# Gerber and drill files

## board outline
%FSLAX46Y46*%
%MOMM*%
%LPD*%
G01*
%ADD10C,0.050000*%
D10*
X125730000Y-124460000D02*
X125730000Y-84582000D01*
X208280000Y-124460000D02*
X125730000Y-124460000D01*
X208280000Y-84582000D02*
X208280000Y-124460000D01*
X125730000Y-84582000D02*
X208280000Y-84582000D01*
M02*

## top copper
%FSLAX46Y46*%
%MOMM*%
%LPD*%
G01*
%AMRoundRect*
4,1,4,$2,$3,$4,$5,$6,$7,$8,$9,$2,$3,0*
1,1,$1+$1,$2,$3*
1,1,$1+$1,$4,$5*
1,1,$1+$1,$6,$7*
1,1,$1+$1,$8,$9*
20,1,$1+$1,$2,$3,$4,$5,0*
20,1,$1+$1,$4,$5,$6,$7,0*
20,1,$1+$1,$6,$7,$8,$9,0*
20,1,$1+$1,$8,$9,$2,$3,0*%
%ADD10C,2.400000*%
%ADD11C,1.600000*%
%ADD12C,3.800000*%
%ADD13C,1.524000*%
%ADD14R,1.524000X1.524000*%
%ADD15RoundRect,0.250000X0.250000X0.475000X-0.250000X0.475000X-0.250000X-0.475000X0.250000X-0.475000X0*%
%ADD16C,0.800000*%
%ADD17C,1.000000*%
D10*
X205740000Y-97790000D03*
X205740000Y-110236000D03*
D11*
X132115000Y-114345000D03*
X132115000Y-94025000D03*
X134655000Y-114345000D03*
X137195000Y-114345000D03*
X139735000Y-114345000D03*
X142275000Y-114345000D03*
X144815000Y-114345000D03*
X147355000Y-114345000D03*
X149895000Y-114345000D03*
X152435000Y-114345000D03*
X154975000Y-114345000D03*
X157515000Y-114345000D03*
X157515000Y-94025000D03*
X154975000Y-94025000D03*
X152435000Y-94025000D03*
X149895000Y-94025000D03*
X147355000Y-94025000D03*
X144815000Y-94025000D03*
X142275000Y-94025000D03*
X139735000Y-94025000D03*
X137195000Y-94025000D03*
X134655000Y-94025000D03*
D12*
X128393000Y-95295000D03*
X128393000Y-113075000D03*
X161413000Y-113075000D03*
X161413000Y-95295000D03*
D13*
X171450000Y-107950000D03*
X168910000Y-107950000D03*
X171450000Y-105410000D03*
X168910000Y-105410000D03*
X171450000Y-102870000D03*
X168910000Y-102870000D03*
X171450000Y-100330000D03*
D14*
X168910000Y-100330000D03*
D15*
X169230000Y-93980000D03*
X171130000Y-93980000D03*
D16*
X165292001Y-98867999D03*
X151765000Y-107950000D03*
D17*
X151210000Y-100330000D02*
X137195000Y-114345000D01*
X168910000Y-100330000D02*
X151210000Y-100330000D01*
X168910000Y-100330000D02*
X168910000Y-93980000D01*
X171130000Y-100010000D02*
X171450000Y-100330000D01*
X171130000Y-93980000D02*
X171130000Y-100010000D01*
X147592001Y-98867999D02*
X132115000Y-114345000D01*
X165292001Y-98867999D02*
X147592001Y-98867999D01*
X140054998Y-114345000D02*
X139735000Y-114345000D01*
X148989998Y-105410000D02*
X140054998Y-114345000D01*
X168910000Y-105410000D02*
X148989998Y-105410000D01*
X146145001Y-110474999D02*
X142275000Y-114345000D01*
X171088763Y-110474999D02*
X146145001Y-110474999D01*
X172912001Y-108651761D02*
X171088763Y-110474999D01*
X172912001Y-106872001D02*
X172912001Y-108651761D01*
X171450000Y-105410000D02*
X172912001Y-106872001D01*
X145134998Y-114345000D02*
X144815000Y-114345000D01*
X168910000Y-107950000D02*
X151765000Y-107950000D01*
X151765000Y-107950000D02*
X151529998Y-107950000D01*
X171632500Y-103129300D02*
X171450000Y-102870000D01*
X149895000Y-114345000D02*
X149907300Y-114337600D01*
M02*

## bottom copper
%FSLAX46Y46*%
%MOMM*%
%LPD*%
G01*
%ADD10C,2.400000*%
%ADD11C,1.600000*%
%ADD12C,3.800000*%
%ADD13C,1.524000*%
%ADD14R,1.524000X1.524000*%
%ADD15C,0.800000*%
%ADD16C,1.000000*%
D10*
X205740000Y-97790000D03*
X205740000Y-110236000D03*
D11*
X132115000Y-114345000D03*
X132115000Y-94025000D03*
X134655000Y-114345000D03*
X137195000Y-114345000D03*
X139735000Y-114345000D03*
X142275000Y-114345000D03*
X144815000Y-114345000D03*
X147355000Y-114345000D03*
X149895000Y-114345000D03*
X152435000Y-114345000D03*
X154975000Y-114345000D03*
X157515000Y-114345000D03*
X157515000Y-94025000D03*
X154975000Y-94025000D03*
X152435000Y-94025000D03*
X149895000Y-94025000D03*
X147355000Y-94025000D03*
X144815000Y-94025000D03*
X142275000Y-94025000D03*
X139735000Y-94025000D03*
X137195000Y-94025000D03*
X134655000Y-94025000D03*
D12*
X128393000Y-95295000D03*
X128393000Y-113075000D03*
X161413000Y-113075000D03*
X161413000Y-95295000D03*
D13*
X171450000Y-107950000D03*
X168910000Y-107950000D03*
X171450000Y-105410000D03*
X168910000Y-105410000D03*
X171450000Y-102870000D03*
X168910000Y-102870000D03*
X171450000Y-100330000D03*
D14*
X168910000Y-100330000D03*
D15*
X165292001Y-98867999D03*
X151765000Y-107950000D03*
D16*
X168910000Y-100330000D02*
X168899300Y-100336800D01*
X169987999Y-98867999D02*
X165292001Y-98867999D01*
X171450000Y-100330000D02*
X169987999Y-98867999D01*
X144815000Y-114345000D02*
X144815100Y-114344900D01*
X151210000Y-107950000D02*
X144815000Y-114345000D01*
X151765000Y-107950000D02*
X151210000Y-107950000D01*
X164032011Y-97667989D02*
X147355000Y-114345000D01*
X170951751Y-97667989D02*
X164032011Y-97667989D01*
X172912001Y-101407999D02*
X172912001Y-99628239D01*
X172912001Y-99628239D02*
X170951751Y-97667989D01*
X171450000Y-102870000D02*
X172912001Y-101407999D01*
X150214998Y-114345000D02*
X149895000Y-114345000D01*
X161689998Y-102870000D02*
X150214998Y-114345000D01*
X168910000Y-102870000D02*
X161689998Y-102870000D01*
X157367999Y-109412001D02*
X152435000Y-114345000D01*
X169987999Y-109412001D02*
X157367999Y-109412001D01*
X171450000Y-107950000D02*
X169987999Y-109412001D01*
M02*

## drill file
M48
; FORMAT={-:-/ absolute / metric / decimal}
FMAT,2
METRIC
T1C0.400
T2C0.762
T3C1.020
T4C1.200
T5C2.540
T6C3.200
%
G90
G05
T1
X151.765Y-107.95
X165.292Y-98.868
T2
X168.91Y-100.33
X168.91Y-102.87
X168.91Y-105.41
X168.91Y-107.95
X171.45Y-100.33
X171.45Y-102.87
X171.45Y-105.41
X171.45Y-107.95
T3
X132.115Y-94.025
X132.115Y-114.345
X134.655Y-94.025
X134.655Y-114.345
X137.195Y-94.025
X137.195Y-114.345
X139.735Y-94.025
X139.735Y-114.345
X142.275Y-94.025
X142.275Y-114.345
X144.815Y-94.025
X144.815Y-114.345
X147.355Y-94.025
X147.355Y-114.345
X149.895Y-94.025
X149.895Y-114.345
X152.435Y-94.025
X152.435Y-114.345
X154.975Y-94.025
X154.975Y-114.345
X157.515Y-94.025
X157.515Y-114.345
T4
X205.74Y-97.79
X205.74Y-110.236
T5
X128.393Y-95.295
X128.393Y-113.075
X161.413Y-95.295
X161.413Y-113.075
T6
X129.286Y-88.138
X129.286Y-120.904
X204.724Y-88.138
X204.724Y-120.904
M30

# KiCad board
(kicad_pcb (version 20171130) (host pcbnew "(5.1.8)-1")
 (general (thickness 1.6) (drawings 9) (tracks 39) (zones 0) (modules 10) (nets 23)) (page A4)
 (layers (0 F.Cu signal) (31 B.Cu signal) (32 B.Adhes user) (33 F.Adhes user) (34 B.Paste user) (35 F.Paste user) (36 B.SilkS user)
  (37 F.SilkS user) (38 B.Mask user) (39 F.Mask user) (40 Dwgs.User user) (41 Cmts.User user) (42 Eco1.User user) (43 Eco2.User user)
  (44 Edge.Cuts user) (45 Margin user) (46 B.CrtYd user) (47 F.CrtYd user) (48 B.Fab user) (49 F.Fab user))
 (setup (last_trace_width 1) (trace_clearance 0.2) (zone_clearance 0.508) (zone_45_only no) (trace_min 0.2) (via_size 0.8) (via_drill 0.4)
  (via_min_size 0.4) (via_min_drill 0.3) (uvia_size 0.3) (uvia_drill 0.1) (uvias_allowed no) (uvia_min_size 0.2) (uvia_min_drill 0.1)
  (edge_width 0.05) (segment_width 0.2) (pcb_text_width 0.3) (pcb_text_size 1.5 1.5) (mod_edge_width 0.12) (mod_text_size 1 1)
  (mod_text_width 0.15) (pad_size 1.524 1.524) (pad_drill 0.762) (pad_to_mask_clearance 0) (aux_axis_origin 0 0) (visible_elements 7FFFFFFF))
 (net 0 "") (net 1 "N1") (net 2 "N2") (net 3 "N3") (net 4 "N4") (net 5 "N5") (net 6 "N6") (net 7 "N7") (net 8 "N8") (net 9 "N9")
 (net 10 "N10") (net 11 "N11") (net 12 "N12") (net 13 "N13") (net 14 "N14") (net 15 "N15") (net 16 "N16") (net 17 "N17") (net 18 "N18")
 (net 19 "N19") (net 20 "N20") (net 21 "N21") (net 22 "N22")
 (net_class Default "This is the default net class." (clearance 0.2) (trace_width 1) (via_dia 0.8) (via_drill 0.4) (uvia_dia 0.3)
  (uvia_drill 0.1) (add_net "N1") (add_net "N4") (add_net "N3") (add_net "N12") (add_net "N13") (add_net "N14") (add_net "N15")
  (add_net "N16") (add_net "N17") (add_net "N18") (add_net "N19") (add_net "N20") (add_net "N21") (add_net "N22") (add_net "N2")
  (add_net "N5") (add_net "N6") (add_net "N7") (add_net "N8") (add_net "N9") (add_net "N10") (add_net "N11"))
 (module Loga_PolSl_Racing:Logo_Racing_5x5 (layer B.Cu) (at 194.31 113.284 90)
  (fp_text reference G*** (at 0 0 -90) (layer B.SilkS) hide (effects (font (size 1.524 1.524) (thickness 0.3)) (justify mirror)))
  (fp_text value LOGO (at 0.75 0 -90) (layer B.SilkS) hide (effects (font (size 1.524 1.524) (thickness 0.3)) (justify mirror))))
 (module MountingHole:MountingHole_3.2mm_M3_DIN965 (layer F.Cu) (at 204.724 120.904)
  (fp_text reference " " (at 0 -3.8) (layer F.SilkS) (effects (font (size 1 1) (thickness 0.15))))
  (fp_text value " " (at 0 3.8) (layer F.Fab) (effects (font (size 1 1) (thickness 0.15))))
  (pad 1 np_thru_hole circle (at 0 0) (size 3.2 3.2) (drill 3.2) (layers *.Cu *.Mask)))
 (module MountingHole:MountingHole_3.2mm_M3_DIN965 (layer F.Cu) (at 129.286 120.904)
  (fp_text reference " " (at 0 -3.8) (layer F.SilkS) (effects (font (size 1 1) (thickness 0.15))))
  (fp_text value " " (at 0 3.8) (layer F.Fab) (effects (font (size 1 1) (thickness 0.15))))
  (pad 1 np_thru_hole circle (at 0 0) (size 3.2 3.2) (drill 3.2) (layers *.Cu *.Mask)))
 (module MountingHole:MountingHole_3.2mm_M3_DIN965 (layer F.Cu) (at 204.724 88.138)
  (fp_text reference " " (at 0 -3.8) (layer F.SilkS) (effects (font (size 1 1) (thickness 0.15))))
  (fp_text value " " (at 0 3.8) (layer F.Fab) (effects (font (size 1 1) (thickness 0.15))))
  (pad 1 np_thru_hole circle (at 0 0) (size 3.2 3.2) (drill 3.2) (layers *.Cu *.Mask)))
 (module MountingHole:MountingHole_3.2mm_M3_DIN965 (layer F.Cu) (at 129.286 88.138)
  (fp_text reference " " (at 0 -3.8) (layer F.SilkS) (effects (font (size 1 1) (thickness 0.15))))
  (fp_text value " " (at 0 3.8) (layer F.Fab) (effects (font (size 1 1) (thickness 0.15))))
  (pad 1 np_thru_hole circle (at 0 0) (size 3.2 3.2) (drill 3.2) (layers *.Cu *.Mask)))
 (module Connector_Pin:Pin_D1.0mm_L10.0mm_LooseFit (layer F.Cu) (at 205.74 97.79)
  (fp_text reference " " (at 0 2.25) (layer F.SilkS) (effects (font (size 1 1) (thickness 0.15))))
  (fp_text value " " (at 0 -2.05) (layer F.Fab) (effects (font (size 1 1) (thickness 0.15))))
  (pad 1 thru_hole circle (at 0 0) (size 2.4 2.4) (drill 1.2) (layers *.Cu *.Mask)))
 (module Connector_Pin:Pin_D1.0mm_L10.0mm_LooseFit (layer F.Cu) (at 205.74 110.236)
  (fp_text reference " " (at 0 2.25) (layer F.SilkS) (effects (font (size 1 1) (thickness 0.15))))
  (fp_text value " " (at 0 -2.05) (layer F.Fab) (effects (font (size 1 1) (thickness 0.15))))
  (pad 1 thru_hole circle (at 0 0) (size 2.4 2.4) (drill 1.2) (layers *.Cu *.Mask)))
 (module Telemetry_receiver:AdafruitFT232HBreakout (layer F.Cu) (at 134.655 114.345)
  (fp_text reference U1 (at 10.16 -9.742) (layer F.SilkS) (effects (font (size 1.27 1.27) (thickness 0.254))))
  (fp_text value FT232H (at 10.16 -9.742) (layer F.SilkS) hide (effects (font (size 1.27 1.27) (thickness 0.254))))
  (pad 0 thru_hole circle (at -2.54 0) (size 1.6 1.6) (drill 1.02) (layers *.Cu *.Mask) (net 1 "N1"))
  (pad 21 thru_hole circle (at -2.54 -20.32) (size 1.6 1.6) (drill 1.02) (layers *.Cu *.Mask) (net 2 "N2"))
  (pad 1 thru_hole circle (at 0 0) (size 1.6 1.6) (drill 1.02) (layers *.Cu *.Mask) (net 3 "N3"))
  (pad 2 thru_hole circle (at 2.54 0) (size 1.6 1.6) (drill 1.02) (layers *.Cu *.Mask) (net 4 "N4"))
  (pad 3 thru_hole circle (at 5.08 0) (size 1.6 1.6) (drill 1.02) (layers *.Cu *.Mask) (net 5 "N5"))
  (pad 4 thru_hole circle (at 7.62 0) (size 1.6 1.6) (drill 1.02) (layers *.Cu *.Mask) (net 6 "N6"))
  (pad 5 thru_hole circle (at 10.16 0) (size 1.6 1.6) (drill 1.02) (layers *.Cu *.Mask) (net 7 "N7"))
  (pad 6 thru_hole circle (at 12.7 0) (size 1.6 1.6) (drill 1.02) (layers *.Cu *.Mask) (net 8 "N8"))
  (pad 7 thru_hole circle (at 15.24 0) (size 1.6 1.6) (drill 1.02) (layers *.Cu *.Mask) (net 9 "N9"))
  (pad 8 thru_hole circle (at 17.78 0) (size 1.6 1.6) (drill 1.02) (layers *.Cu *.Mask) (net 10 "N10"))
  (pad 9 thru_hole circle (at 20.32 0) (size 1.6 1.6) (drill 1.02) (layers *.Cu *.Mask) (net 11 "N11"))
  (pad 10 thru_hole circle (at 22.86 0) (size 1.6 1.6) (drill 1.02) (layers *.Cu *.Mask) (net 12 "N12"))
  (pad 11 thru_hole circle (at 22.86 -20.32) (size 1.6 1.6) (drill 1.02) (layers *.Cu *.Mask) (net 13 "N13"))
  (pad 12 thru_hole circle (at 20.32 -20.32) (size 1.6 1.6) (drill 1.02) (layers *.Cu *.Mask) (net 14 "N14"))
  (pad 13 thru_hole circle (at 17.78 -20.32) (size 1.6 1.6) (drill 1.02) (layers *.Cu *.Mask) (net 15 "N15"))
  (pad 14 thru_hole circle (at 15.24 -20.32) (size 1.6 1.6) (drill 1.02) (layers *.Cu *.Mask) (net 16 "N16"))
  (pad 15 thru_hole circle (at 12.7 -20.32) (size 1.6 1.6) (drill 1.02) (layers *.Cu *.Mask) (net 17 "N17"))
  (pad 16 thru_hole circle (at 10.16 -20.32) (size 1.6 1.6) (drill 1.02) (layers *.Cu *.Mask) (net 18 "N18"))
  (pad 17 thru_hole circle (at 7.62 -20.32) (size 1.6 1.6) (drill 1.02) (layers *.Cu *.Mask) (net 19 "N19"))
  (pad 18 thru_hole circle (at 5.08 -20.32) (size 1.6 1.6) (drill 1.02) (layers *.Cu *.Mask) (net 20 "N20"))
  (pad 19 thru_hole circle (at 2.54 -20.32) (size 1.6 1.6) (drill 1.02) (layers *.Cu *.Mask) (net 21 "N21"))
  (pad 20 thru_hole circle (at 0 -20.32) (size 1.6 1.6) (drill 1.02) (layers *.Cu *.Mask) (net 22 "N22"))
  (pad 25 thru_hole circle (at -6.262 -19.05) (size 3.8 3.8) (drill 2.54) (layers *.Cu *.Mask))
  (pad 22 thru_hole circle (at -6.262 -1.27) (size 3.8 3.8) (drill 2.54) (layers *.Cu *.Mask))
  (pad 23 thru_hole circle (at 26.758 -1.27) (size 3.8 3.8) (drill 2.54) (layers *.Cu *.Mask))
  (pad 24 thru_hole circle (at 26.758 -19.05) (size 3.8 3.8) (drill 2.54) (layers *.Cu *.Mask)))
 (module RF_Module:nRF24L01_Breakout (layer F.Cu) (at 168.91 100.33)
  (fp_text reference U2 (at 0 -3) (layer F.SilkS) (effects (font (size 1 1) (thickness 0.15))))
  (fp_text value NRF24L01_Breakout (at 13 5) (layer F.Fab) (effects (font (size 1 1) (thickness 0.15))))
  (pad 8 thru_hole circle (at 2.54 7.62) (size 1.524 1.524) (drill 0.762) (layers *.Cu *.Mask) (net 10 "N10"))
  (pad 7 thru_hole circle (at 0 7.62) (size 1.524 1.524) (drill 0.762) (layers *.Cu *.Mask) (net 7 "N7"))
  (pad 6 thru_hole circle (at 2.54 5.08) (size 1.524 1.524) (drill 0.762) (layers *.Cu *.Mask) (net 6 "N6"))
  (pad 5 thru_hole circle (at 0 5.08) (size 1.524 1.524) (drill 0.762) (layers *.Cu *.Mask) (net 5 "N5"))
  (pad 4 thru_hole circle (at 2.54 2.54) (size 1.524 1.524) (drill 0.762) (layers *.Cu *.Mask) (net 8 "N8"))
  (pad 3 thru_hole circle (at 0 2.54) (size 1.524 1.524) (drill 0.762) (layers *.Cu *.Mask) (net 9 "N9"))
  (pad 2 thru_hole circle (at 2.54 0) (size 1.524 1.524) (drill 0.762) (layers *.Cu *.Mask) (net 1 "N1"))
  (pad 1 thru_hole rect (at 0 0) (size 1.524 1.524) (drill 0.762) (layers *.Cu *.Mask) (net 4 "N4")))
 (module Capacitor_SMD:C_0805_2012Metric (layer F.Cu) (at 170.18 93.98 180)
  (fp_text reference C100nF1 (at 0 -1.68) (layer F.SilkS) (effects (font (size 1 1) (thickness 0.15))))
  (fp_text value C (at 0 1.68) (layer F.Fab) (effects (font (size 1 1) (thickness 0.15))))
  (pad 2 smd roundrect (at 0.95 0 180) (size 1 1.45) (layers F.Cu F.Paste F.Mask) (roundrect_rratio 0.25) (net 4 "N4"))
  (pad 1 smd roundrect (at -0.95 0 180) (size 1 1.45) (layers F.Cu F.Paste F.Mask) (roundrect_rratio 0.25) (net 1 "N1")))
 (gr_line (start 125.73 124.46) (end 125.73 84.582) (layer Edge.Cuts) (width 0.05))
 (gr_line (start 208.28 124.46) (end 125.73 124.46) (layer Edge.Cuts) (width 0.05))
 (gr_line (start 208.28 84.582) (end 208.28 124.46) (layer Edge.Cuts) (width 0.05))
 (gr_line (start 125.73 84.582) (end 208.28 84.582) (layer Edge.Cuts) (width 0.05))
 (segment (start 168.91 100.33) (end 168.8993 100.3368) (width 1) (layer B.Cu) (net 4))
 (segment (start 151.21 100.33) (end 137.195 114.345) (width 1) (layer F.Cu) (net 4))
 (segment (start 168.91 100.33) (end 151.21 100.33) (width 1) (layer F.Cu) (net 4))
 (segment (start 168.91 100.33) (end 168.91 93.98) (width 1) (layer F.Cu) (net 4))
 (segment (start 171.13 100.01) (end 171.45 100.33) (width 1) (layer F.Cu) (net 1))
 (segment (start 171.13 93.98) (end 171.13 100.01) (width 1) (layer F.Cu) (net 1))
 (segment (start 169.987999 98.867999) (end 165.292001 98.867999) (width 1) (layer B.Cu) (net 1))
 (segment (start 171.45 100.33) (end 169.987999 98.867999) (width 1) (layer B.Cu) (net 1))
 (via (at 165.292001 98.867999) (size 0.8) (drill 0.4) (layers F.Cu B.Cu) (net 1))
 (segment (start 147.592001 98.867999) (end 132.115 114.345) (width 1) (layer F.Cu) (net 1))
 (segment (start 165.292001 98.867999) (end 147.592001 98.867999) (width 1) (layer F.Cu) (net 1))
 (segment (start 140.054998 114.345) (end 139.735 114.345) (width 1) (layer F.Cu) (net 5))
 (segment (start 148.989998 105.41) (end 140.054998 114.345) (width 1) (layer F.Cu) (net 5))
 (segment (start 168.91 105.41) (end 148.989998 105.41) (width 1) (layer F.Cu) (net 5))
 (segment (start 146.145001 110.474999) (end 142.275 114.345) (width 1) (layer F.Cu) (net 6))
 (segment (start 171.088763 110.474999) (end 146.145001 110.474999) (width 1) (layer F.Cu) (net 6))
 (segment (start 172.912001 108.651761) (end 171.088763 110.474999) (width 1) (layer F.Cu) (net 6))
 (segment (start 172.912001 106.872001) (end 172.912001 108.651761) (width 1) (layer F.Cu) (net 6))
 (segment (start 171.45 105.41) (end 172.912001 106.872001) (width 1) (layer F.Cu) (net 6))
 (segment (start 144.815 114.345) (end 144.8151 114.3449) (width 1) (layer B.Cu) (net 7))
 (segment (start 145.134998 114.345) (end 144.815 114.345) (width 1) (layer F.Cu) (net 7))
 (segment (start 168.91 107.95) (end 151.765 107.95) (width 1) (layer F.Cu) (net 7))
 (segment (start 151.765 107.95) (end 151.529998 107.95) (width 1) (layer F.Cu) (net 7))
 (via (at 151.765 107.95) (size 0.8) (drill 0.4) (layers F.Cu B.Cu) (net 7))
 (segment (start 151.21 107.95) (end 144.815 114.345) (width 1) (layer B.Cu) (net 7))
 (segment (start 151.765 107.95) (end 151.21 107.95) (width 1) (layer B.Cu) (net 7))
 (segment (start 171.6325 103.1293) (end 171.45 102.87) (width 1) (layer F.Cu) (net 8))
 (segment (start 164.032011 97.667989) (end 147.355 114.345) (width 1) (layer B.Cu) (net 8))
 (segment (start 170.951751 97.667989) (end 164.032011 97.667989) (width 1) (layer B.Cu) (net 8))
 (segment (start 172.912001 101.407999) (end 172.912001 99.628239) (width 1) (layer B.Cu) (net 8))
 (segment (start 172.912001 99.628239) (end 170.951751 97.667989) (width 1) (layer B.Cu) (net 8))
 (segment (start 171.45 102.87) (end 172.912001 101.407999) (width 1) (layer B.Cu) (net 8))
 (segment (start 149.895 114.345) (end 149.9073 114.3376) (width 1) (layer F.Cu) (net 9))
 (segment (start 150.214998 114.345) (end 149.895 114.345) (width 1) (layer B.Cu) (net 9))
 (segment (start 161.689998 102.87) (end 150.214998 114.345) (width 1) (layer B.Cu) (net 9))
 (segment (start 168.91 102.87) (end 161.689998 102.87) (width 1) (layer B.Cu) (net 9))
 (segment (start 157.367999 109.412001) (end 152.435 114.345) (width 1) (layer B.Cu) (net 10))
 (segment (start 169.987999 109.412001) (end 157.367999 109.412001) (width 1) (layer B.Cu) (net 10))
 (segment (start 171.45 107.95) (end 169.987999 109.412001) (width 1) (layer B.Cu) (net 10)))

